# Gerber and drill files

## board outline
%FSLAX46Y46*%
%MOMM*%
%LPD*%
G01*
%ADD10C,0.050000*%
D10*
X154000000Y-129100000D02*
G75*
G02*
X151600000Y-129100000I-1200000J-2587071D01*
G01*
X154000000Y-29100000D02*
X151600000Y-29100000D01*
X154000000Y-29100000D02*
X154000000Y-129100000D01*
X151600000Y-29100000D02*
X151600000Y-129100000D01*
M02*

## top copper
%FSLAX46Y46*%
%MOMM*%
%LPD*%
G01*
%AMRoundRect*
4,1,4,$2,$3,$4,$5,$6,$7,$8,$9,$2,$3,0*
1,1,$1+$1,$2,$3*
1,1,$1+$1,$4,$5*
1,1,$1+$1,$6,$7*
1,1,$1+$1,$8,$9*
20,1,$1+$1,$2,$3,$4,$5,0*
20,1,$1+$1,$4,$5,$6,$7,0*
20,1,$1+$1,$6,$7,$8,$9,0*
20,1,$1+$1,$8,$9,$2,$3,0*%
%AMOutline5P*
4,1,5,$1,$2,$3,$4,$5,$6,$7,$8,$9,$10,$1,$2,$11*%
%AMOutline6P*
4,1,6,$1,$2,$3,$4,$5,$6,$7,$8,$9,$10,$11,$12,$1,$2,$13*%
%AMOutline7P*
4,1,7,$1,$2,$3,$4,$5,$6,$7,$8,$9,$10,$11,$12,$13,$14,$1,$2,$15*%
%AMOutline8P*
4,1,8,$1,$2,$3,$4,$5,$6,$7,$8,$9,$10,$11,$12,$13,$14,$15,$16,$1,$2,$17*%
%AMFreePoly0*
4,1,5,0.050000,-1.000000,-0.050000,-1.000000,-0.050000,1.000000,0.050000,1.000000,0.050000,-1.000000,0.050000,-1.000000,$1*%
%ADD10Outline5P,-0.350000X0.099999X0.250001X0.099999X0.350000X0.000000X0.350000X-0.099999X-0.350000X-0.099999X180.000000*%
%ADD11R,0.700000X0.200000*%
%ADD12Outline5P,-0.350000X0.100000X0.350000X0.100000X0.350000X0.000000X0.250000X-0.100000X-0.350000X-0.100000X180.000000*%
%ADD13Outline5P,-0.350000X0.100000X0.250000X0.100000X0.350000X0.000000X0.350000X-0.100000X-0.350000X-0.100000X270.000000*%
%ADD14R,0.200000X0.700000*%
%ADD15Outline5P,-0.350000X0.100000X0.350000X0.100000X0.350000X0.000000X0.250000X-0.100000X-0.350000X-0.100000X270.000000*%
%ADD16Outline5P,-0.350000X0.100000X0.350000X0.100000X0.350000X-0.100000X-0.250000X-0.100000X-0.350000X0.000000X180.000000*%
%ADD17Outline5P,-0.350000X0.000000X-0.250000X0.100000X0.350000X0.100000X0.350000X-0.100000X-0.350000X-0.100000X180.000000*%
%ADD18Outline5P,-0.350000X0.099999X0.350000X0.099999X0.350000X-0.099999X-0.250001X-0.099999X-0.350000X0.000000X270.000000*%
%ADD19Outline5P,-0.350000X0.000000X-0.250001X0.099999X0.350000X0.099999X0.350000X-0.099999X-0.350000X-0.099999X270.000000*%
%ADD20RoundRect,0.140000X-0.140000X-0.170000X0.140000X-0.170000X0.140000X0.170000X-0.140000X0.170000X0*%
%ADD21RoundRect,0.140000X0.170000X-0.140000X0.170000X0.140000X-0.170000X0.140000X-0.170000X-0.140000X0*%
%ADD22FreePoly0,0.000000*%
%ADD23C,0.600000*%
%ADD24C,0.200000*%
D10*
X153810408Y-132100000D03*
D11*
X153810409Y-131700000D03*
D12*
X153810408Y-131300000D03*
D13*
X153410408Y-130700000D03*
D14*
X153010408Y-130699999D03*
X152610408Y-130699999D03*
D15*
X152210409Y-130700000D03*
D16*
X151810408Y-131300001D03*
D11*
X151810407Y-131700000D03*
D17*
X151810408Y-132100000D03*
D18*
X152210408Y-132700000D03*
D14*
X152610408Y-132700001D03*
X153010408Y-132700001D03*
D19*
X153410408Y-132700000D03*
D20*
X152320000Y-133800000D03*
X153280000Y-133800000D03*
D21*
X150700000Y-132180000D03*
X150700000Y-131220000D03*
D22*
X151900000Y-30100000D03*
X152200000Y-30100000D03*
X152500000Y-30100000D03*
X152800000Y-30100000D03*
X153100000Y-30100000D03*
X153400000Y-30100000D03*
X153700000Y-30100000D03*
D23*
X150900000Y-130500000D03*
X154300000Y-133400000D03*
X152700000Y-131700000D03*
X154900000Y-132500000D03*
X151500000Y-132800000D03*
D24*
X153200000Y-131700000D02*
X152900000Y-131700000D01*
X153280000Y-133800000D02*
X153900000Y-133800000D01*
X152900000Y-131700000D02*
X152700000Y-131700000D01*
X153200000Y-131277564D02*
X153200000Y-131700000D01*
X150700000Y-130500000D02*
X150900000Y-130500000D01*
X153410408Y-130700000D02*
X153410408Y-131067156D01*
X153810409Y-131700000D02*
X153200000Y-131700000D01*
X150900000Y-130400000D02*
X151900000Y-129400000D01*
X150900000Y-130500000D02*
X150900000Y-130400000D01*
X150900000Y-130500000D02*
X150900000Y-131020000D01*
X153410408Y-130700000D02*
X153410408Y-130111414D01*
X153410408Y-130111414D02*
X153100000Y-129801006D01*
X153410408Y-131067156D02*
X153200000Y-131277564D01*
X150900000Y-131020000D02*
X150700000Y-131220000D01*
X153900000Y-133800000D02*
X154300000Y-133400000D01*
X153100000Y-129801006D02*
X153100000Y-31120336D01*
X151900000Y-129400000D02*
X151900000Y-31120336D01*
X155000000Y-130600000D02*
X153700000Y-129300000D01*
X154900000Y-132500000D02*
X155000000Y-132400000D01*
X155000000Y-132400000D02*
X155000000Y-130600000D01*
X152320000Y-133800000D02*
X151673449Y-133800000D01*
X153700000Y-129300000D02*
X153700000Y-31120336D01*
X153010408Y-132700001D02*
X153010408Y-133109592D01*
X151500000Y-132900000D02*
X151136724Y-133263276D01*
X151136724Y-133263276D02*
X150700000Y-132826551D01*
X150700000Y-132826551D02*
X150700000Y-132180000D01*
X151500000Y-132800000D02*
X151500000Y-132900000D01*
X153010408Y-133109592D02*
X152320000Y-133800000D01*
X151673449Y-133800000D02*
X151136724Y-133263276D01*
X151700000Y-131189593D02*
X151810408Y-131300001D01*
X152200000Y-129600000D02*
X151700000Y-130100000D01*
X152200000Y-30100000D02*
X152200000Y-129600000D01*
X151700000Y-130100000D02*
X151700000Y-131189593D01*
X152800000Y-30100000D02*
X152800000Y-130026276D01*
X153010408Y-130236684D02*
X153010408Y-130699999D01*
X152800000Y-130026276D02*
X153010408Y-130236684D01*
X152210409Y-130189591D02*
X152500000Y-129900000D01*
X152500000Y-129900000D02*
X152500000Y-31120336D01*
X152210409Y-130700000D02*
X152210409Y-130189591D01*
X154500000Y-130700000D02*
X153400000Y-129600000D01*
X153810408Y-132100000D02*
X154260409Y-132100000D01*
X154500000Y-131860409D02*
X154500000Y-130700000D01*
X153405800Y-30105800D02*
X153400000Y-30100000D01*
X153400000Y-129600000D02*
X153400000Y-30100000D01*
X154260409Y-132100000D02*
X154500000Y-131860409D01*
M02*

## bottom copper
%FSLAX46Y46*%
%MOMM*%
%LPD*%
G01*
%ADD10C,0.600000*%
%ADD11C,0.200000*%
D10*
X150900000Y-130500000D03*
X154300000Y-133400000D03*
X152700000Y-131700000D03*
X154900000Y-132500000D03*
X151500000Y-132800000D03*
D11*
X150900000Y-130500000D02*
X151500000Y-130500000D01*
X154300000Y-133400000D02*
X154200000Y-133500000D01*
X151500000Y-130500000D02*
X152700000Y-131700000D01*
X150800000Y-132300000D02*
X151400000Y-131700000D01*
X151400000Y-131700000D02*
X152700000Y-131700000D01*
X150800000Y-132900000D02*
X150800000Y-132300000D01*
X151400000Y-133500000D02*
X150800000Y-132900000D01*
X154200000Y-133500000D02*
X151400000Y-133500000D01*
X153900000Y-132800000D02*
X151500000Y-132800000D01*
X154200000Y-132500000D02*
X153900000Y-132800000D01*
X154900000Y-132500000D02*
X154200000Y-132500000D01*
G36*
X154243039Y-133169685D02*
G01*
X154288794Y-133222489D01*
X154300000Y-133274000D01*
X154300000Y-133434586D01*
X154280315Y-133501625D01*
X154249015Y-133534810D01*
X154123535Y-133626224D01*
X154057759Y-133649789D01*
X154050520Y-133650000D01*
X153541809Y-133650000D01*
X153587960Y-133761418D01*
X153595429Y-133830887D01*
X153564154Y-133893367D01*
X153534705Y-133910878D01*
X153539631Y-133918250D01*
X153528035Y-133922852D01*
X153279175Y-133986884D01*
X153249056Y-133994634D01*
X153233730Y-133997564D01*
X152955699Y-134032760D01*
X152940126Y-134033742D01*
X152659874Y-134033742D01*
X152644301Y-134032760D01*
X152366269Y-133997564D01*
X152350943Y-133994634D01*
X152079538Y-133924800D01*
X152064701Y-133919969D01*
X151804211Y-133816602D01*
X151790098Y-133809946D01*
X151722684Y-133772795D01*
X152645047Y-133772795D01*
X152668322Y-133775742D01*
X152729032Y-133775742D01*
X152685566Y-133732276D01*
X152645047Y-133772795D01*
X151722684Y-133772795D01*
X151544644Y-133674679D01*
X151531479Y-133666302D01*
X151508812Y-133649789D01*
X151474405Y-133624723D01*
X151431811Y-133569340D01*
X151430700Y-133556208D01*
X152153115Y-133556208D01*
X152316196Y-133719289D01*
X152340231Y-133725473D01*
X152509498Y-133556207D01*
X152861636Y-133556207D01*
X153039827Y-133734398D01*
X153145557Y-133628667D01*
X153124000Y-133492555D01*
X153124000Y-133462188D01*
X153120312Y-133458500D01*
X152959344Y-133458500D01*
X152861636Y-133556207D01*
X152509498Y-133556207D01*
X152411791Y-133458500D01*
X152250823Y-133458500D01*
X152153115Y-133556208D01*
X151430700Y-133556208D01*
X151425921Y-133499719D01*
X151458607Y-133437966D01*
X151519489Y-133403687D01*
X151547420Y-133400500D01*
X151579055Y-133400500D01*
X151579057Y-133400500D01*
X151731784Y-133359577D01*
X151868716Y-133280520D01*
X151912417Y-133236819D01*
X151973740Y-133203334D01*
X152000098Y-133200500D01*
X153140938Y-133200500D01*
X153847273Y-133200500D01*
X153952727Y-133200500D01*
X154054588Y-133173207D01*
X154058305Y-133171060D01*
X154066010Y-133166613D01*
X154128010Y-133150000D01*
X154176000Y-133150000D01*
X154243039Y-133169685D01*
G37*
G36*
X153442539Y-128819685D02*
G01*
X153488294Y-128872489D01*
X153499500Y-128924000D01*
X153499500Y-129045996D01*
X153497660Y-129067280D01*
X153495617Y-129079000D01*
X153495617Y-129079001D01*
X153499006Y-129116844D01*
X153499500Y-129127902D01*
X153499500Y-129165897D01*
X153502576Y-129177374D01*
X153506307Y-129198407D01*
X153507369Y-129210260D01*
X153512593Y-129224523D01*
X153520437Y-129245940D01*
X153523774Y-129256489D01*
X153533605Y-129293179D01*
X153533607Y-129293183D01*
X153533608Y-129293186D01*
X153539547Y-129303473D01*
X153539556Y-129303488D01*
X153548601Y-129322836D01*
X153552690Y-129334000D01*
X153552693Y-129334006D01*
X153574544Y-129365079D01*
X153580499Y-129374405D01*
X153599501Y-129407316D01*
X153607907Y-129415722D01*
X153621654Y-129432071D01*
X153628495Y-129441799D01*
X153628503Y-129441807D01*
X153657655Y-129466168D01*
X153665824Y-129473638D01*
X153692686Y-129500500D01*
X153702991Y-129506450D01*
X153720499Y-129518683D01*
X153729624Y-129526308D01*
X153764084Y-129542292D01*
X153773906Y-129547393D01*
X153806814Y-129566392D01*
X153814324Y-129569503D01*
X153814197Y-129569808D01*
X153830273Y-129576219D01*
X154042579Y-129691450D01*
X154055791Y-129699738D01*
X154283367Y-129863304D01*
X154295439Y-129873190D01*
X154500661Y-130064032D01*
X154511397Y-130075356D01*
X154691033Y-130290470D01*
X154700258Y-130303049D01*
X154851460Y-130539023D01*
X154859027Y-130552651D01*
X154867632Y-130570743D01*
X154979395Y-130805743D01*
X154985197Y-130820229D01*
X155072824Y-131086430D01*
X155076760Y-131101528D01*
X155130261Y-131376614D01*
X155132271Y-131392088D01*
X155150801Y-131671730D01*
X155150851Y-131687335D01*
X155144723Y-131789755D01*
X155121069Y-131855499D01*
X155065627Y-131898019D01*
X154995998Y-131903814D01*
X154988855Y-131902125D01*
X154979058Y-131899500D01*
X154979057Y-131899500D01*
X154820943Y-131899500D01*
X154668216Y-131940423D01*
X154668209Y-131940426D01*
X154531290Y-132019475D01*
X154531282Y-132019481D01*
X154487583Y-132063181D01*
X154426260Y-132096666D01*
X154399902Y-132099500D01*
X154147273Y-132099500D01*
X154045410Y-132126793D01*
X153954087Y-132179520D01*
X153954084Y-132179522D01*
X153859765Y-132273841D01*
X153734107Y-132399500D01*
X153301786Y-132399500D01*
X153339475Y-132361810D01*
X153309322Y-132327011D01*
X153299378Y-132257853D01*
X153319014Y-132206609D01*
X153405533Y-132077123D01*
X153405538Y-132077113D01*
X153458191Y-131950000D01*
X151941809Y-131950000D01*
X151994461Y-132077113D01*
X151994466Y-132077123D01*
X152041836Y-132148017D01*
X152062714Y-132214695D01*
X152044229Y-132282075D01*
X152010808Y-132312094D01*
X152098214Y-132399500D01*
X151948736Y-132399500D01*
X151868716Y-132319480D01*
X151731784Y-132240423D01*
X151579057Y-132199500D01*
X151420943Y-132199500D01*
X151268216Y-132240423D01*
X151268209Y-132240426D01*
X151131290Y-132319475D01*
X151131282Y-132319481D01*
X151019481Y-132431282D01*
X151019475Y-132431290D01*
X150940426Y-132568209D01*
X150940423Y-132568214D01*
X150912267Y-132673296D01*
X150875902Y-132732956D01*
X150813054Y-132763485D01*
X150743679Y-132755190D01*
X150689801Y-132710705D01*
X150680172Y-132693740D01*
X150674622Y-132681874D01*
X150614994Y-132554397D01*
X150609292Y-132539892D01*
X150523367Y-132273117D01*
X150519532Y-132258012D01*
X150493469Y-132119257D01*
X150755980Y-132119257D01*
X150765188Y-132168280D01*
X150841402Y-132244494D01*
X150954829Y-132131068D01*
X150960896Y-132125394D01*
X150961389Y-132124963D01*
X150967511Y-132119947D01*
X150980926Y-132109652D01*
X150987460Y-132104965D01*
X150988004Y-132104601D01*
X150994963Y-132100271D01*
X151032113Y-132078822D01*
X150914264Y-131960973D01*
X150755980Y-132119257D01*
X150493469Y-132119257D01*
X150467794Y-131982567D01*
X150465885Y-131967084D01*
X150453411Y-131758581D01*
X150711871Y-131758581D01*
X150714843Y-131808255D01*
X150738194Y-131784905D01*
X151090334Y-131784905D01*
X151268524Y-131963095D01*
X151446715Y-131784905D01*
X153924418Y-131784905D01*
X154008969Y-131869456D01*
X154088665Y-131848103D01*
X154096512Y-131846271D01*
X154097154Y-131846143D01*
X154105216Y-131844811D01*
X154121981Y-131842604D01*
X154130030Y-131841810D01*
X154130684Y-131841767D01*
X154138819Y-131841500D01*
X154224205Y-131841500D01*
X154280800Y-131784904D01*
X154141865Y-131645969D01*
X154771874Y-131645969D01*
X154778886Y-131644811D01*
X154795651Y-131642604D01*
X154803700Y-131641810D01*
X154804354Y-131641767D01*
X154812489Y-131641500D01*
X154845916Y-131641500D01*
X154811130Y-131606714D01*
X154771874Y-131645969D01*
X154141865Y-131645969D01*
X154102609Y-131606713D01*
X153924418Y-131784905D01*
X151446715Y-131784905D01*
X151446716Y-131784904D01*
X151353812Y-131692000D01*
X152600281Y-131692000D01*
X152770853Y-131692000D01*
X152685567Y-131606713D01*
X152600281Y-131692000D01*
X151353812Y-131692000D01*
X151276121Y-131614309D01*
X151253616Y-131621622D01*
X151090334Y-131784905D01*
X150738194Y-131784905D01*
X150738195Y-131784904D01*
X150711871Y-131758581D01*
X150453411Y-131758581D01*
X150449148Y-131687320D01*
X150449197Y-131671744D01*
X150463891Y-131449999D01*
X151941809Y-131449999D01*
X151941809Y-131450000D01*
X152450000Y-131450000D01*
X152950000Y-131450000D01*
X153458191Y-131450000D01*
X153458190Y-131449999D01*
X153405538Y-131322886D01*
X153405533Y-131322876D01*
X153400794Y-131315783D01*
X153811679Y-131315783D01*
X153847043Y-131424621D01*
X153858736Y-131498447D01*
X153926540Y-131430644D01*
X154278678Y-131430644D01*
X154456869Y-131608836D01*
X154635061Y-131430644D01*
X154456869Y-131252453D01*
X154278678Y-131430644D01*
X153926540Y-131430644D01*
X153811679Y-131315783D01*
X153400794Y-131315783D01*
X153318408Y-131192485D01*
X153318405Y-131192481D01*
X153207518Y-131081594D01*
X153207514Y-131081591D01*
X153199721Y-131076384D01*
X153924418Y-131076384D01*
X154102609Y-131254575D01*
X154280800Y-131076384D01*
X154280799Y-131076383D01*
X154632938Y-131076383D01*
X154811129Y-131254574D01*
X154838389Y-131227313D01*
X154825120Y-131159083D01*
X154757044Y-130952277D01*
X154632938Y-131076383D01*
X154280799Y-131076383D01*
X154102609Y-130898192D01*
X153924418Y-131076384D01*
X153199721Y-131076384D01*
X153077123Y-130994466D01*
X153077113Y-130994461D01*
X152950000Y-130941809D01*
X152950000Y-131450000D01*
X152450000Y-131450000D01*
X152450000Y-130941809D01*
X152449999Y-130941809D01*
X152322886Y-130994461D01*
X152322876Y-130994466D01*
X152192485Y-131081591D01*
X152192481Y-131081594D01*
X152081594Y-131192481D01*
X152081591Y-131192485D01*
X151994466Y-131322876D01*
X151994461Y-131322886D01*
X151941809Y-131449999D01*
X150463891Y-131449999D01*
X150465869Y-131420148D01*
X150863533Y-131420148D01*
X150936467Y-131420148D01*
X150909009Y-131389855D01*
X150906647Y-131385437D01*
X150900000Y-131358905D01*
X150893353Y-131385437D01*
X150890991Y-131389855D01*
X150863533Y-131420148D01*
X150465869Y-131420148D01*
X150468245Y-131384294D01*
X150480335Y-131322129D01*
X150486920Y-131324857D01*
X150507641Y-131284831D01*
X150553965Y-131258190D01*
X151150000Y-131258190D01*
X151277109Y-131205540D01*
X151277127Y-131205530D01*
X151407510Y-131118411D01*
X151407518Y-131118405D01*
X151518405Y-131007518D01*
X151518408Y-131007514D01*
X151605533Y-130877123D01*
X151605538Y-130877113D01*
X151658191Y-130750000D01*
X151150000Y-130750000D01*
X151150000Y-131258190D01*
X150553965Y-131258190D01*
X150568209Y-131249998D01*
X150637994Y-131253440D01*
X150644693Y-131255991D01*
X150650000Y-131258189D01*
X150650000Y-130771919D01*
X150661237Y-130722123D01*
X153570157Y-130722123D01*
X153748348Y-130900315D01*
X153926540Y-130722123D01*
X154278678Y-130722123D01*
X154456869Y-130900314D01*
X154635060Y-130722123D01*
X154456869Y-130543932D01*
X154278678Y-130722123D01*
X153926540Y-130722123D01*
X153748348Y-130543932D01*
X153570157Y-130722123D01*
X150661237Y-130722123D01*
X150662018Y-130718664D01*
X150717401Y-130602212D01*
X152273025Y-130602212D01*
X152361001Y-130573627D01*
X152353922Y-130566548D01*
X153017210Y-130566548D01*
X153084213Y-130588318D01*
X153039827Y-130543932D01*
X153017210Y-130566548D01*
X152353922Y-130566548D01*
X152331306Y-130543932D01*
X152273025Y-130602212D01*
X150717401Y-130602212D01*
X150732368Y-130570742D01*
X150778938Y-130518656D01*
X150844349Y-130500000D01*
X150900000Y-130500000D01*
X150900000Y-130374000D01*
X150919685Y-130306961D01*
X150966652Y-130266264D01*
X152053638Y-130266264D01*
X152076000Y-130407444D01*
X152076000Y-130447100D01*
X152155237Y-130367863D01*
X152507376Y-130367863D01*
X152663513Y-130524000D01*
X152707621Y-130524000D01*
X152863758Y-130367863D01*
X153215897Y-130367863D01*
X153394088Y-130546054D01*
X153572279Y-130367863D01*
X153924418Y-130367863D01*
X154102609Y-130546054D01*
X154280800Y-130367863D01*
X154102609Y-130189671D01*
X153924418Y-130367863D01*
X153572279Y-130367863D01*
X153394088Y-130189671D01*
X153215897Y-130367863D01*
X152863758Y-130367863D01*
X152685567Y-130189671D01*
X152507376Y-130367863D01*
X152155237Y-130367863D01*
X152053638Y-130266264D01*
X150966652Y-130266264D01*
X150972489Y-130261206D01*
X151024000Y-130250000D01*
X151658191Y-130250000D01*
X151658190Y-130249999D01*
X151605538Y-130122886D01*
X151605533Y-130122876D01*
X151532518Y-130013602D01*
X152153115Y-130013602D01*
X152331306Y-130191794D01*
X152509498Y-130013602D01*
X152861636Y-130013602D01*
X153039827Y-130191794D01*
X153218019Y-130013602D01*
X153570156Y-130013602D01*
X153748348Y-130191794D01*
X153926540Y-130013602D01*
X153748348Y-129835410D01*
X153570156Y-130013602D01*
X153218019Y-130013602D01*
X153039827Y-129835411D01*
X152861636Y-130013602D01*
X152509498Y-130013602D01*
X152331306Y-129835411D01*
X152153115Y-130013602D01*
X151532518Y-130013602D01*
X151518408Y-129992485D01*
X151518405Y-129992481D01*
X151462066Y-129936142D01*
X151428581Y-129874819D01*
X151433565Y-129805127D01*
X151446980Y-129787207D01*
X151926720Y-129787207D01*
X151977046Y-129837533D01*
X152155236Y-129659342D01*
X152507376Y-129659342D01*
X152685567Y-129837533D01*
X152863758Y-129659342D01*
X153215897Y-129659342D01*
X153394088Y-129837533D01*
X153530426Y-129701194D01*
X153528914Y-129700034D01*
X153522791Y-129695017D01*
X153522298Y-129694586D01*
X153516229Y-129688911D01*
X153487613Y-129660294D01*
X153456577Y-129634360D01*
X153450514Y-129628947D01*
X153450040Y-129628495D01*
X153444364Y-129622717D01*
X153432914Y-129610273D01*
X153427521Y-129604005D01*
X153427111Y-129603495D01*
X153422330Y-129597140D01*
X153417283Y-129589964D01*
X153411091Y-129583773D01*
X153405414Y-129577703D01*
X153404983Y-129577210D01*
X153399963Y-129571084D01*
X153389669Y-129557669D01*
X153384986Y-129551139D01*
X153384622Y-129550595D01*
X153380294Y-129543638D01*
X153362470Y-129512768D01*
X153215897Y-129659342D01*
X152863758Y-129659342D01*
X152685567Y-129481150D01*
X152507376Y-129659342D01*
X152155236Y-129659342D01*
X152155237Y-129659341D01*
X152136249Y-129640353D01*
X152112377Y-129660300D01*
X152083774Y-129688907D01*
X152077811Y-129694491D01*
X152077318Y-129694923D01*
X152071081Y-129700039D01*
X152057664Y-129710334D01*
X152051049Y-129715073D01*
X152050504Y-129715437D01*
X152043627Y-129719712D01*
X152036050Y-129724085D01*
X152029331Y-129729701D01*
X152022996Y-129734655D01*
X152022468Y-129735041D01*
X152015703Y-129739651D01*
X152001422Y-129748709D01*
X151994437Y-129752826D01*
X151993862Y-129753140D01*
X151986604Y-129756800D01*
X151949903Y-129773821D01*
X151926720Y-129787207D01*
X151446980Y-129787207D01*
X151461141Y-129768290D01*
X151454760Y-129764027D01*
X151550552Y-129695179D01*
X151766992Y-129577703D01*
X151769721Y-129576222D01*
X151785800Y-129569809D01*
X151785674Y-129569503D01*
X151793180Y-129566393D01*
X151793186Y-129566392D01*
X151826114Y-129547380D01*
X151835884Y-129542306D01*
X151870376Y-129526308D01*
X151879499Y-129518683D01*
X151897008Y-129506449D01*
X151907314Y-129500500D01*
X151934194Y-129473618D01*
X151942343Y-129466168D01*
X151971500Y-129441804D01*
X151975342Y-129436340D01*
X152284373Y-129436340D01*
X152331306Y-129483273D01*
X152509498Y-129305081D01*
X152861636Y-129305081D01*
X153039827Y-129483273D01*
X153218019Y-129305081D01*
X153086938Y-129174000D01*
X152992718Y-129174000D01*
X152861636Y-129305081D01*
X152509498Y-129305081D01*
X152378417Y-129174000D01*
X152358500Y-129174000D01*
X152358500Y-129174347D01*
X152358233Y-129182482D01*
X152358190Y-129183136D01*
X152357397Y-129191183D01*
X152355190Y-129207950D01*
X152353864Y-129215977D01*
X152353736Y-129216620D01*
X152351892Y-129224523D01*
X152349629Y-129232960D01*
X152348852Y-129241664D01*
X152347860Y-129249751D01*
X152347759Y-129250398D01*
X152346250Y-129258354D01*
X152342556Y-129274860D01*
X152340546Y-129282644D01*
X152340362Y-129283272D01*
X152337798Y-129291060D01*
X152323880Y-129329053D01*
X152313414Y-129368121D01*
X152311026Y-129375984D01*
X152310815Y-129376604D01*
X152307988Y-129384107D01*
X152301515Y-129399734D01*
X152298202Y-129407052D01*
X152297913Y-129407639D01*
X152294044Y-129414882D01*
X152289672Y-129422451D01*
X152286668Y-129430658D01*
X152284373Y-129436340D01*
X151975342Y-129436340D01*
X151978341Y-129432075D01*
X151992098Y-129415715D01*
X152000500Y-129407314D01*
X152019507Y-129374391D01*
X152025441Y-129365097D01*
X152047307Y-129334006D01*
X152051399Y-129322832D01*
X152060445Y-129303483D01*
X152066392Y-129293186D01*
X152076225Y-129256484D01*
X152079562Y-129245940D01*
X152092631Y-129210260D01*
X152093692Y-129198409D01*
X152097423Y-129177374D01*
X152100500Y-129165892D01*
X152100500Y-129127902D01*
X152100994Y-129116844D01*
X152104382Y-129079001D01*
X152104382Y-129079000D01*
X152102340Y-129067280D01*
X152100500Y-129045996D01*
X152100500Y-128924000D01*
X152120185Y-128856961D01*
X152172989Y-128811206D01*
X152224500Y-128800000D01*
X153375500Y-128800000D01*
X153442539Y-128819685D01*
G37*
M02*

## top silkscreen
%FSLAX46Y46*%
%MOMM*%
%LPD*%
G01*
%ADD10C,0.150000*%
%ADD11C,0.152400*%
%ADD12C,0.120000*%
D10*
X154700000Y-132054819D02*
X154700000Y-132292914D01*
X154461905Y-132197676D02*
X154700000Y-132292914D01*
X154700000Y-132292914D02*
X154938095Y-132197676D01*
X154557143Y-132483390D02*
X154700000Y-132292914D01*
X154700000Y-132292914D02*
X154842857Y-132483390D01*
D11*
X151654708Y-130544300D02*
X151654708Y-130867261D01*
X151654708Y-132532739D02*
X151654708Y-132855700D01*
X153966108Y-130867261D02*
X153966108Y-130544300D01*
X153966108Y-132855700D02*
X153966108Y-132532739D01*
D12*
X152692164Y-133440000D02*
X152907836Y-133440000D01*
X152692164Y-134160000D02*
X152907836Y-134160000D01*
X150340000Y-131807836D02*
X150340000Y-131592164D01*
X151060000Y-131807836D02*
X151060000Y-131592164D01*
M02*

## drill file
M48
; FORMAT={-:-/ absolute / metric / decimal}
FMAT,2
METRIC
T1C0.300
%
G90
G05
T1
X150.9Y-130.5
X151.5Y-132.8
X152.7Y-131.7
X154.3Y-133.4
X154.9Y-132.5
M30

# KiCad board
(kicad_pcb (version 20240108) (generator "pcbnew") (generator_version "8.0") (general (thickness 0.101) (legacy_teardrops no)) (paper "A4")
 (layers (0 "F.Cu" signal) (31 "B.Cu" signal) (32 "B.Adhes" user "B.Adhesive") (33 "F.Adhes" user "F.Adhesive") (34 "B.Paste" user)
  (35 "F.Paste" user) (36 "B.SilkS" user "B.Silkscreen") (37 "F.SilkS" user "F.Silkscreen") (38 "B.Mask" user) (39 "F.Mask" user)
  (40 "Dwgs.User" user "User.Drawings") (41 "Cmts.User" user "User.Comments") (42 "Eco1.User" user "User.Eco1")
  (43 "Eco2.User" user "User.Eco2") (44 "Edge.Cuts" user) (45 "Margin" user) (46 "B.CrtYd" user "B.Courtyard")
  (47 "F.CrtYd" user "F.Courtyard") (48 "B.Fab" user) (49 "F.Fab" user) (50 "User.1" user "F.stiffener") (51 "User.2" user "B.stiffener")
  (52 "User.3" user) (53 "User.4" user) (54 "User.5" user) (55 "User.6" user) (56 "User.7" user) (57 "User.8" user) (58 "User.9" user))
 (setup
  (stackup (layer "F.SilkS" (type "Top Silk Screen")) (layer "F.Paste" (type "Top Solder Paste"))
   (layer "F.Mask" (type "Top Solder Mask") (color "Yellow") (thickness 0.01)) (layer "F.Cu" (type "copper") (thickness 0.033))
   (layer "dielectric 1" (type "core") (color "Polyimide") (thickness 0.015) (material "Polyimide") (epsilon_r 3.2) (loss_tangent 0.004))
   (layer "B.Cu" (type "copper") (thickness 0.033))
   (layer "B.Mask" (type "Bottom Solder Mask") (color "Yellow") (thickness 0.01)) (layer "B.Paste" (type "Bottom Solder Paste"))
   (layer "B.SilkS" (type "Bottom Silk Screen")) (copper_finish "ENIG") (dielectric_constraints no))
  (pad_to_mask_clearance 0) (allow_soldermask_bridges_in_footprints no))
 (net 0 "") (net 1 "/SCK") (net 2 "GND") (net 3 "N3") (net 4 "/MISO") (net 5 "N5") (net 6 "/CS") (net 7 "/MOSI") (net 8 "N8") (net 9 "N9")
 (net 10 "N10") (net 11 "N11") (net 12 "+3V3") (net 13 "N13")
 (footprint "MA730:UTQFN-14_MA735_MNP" (layer "F.Cu") (at 152.810408 131.7 180)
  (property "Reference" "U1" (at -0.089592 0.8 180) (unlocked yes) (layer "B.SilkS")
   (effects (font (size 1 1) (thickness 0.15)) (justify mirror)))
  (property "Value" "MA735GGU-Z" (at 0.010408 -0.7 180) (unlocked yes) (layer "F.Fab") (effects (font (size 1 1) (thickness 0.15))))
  (fp_line (start 1.1557 1.1557) (end 1.1557 0.832739) (stroke (width 0.1524) (type solid)) (layer "F.SilkS"))
  (fp_line (start 1.1557 -0.832739) (end 1.1557 -1.1557) (stroke (width 0.1524) (type solid)) (layer "F.SilkS"))
  (fp_line (start -1.1557 0.832739) (end -1.1557 1.1557) (stroke (width 0.1524) (type solid)) (layer "F.SilkS"))
  (fp_line (start -1.1557 -1.1557) (end -1.1557 -0.832739) (stroke (width 0.1524) (type solid)) (layer "F.SilkS"))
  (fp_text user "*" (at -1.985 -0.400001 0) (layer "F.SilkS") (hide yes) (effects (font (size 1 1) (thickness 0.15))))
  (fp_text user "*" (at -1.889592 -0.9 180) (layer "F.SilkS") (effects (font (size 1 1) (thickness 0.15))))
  (pad "1" smd roundrect (at -1 -0.4 180) (size 0.7 0.199998) (layers "F.Cu" "F.Paste" "F.Mask") (roundrect_rratio 0) (chamfer_ratio 0.5)
   (chamfer top_right) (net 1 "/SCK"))
  (pad "2" smd rect (at -1.000001 0 180) (size 0.7 0.2) (layers "F.Cu" "F.Paste" "F.Mask") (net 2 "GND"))
  (pad "3" smd roundrect (at -1 0.4 180) (size 0.7 0.2) (layers "F.Cu" "F.Paste" "F.Mask") (roundrect_rratio 0) (chamfer_ratio 0.5)
   (chamfer bottom_right) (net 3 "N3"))
  (pad "4" smd roundrect (at -0.6 1 270) (size 0.7 0.2) (layers "F.Cu" "F.Paste" "F.Mask") (roundrect_rratio 0) (chamfer_ratio 0.5)
   (chamfer top_right) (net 2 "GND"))
  (pad "5" smd rect (at -0.2 1.000001 270) (size 0.7 0.2) (layers "F.Cu" "F.Paste" "F.Mask") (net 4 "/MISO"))
  (pad "6" smd rect (at 0.2 1.000001 270) (size 0.7 0.2) (layers "F.Cu" "F.Paste" "F.Mask") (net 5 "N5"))
  (pad "7" smd roundrect (at 0.599999 1 270) (size 0.7 0.199999) (layers "F.Cu" "F.Paste" "F.Mask") (roundrect_rratio 0) (chamfer_ratio 0.5)
   (chamfer bottom_right) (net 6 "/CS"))
  (pad "8" smd roundrect (at 1 0.399999 180) (size 0.7 0.2) (layers "F.Cu" "F.Paste" "F.Mask") (roundrect_rratio 0) (chamfer_ratio 0.5)
   (chamfer bottom_left) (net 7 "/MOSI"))
  (pad "9" smd rect (at 1.000001 0 180) (size 0.7 0.2) (layers "F.Cu" "F.Paste" "F.Mask") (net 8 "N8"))
  (pad "10" smd roundrect (at 1 -0.4 180) (size 0.7 0.2) (layers "F.Cu" "F.Paste" "F.Mask") (roundrect_rratio 0) (chamfer_ratio 0.5)
   (chamfer top_left) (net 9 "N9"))
  (pad "11" smd roundrect (at 0.6 -1 270) (size 0.7 0.199998) (layers "F.Cu" "F.Paste" "F.Mask") (roundrect_rratio 0) (chamfer_ratio 0.5)
   (chamfer bottom_left) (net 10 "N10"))
  (pad "12" smd rect (at 0.2 -1.000001 270) (size 0.7 0.2) (layers "F.Cu" "F.Paste" "F.Mask") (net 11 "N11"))
  (pad "13" smd rect (at -0.2 -1.000001 270) (size 0.7 0.2) (layers "F.Cu" "F.Paste" "F.Mask") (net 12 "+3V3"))
  (pad "14" smd roundrect (at -0.6 -1 270) (size 0.7 0.199998) (layers "F.Cu" "F.Paste" "F.Mask") (roundrect_rratio 0) (chamfer_ratio 0.5)
   (chamfer top_left) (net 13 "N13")))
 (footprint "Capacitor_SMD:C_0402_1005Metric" (layer "F.Cu") (at 152.8 133.8)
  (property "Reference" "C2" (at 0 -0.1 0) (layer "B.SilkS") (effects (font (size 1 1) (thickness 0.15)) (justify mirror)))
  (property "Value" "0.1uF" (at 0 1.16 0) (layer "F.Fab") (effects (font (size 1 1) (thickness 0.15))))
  (fp_line (start -0.107836 -0.36) (end 0.107836 -0.36) (stroke (width 0.12) (type solid)) (layer "F.SilkS"))
  (fp_line (start -0.107836 0.36) (end 0.107836 0.36) (stroke (width 0.12) (type solid)) (layer "F.SilkS"))
  (pad "1" smd roundrect (at -0.48 0) (size 0.56 0.62) (layers "F.Cu" "F.Paste" "F.Mask") (roundrect_rratio 0.25) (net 12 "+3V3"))
  (pad "2" smd roundrect (at 0.48 0) (size 0.56 0.62) (layers "F.Cu" "F.Paste" "F.Mask") (roundrect_rratio 0.25) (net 2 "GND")))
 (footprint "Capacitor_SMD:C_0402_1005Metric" (layer "F.Cu") (at 150.7 131.7 90)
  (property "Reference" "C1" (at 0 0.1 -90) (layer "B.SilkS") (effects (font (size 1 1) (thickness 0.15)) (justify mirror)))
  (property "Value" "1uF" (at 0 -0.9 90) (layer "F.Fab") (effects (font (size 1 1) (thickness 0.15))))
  (fp_line (start -0.107836 -0.36) (end 0.107836 -0.36) (stroke (width 0.12) (type solid)) (layer "F.SilkS"))
  (fp_line (start -0.107836 0.36) (end 0.107836 0.36) (stroke (width 0.12) (type solid)) (layer "F.SilkS"))
  (pad "1" smd roundrect (at -0.48 0 90) (size 0.56 0.62) (layers "F.Cu" "F.Paste" "F.Mask") (roundrect_rratio 0.25) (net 12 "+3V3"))
  (pad "2" smd roundrect (at 0.48 0 90) (size 0.56 0.62) (layers "F.Cu" "F.Paste" "F.Mask") (roundrect_rratio 0.25) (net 2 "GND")))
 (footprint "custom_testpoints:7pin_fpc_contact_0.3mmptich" (layer "F.Cu") (at 152.8 30.2)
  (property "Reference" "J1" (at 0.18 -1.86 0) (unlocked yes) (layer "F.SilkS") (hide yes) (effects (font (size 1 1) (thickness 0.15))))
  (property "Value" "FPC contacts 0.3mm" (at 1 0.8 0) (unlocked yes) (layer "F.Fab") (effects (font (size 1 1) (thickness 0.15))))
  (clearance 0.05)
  (pad "1" connect custom (at -0.9 -0.1) (size 0.1 2) (layers "F.Cu" "F.Mask") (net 2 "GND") (clearance 0.05)
   (options (clearance outline) (anchor rect)) (primitives))
  (pad "2" connect custom (at -0.6 -0.1) (size 0.1 2) (layers "F.Cu" "F.Mask") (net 7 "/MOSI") (clearance 0.05)
   (options (clearance outline) (anchor rect)) (primitives))
  (pad "3" connect custom (at -0.3 -0.1) (size 0.1 2) (layers "F.Cu" "F.Mask") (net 6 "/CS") (clearance 0.05)
   (options (clearance outline) (anchor rect)) (primitives))
  (pad "4" connect custom (at 0 -0.1) (size 0.1 2) (layers "F.Cu" "F.Mask") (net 4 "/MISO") (clearance 0.05)
   (options (clearance outline) (anchor rect)) (primitives))
  (pad "5" connect custom (at 0.3 -0.1) (size 0.1 2) (layers "F.Cu" "F.Mask") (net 2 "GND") (clearance 0.05)
   (options (clearance outline) (anchor rect)) (primitives))
  (pad "6" connect custom (at 0.6 -0.1) (size 0.1 2) (layers "F.Cu" "F.Mask") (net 1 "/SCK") (clearance 0.05)
   (options (clearance outline) (anchor rect)) (primitives))
  (pad "7" connect custom (at 0.9 -0.1) (size 0.1 2) (layers "F.Cu" "F.Mask") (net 12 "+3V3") (clearance 0.05)
   (options (clearance outline) (anchor rect)) (primitives)))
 (gr_arc (start 154 129.1) (mid 152.8 134.538901) (end 151.6 129.1) (stroke (width 0.05) (type default)) (layer "Edge.Cuts"))
 (gr_line (start 154 29.1) (end 151.6 29.1) (stroke (width 0.05) (type default)) (layer "Edge.Cuts"))
 (gr_line (start 154 29.1) (end 154 129.1) (stroke (width 0.05) (type default)) (layer "Edge.Cuts"))
 (gr_line (start 151.6 29.1) (end 151.6 129.1) (stroke (width 0.05) (type default)) (layer "Edge.Cuts"))
 (segment (start 153.2 131.7) (end 152.9 131.7) (width 0.2) (layer "F.Cu") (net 2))
 (segment (start 153.28 133.8) (end 153.9 133.8) (width 0.2) (layer "F.Cu") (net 2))
 (segment (start 152.9 131.7) (end 152.7 131.7) (width 0.2) (layer "F.Cu") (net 2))
 (segment (start 153.2 131.277564) (end 153.2 131.7) (width 0.2) (layer "F.Cu") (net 2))
 (segment (start 150.7 130.5) (end 150.9 130.5) (width 0.2) (layer "F.Cu") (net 2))
 (segment (start 153.410408 130.7) (end 153.410408 131.067156) (width 0.2) (layer "F.Cu") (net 2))
 (segment (start 153.810409 131.7) (end 153.2 131.7) (width 0.2) (layer "F.Cu") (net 2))
 (segment (start 150.9 130.4) (end 151.9 129.4) (width 0.2) (layer "F.Cu") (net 2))
 (segment (start 150.9 130.5) (end 150.9 130.4) (width 0.2) (layer "F.Cu") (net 2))
 (segment (start 150.9 130.5) (end 150.9 131.02) (width 0.2) (layer "F.Cu") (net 2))
 (segment (start 153.410408 130.7) (end 153.410408 130.111414) (width 0.2) (layer "F.Cu") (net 2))
 (segment (start 153.410408 130.111414) (end 153.1 129.801006) (width 0.2) (layer "F.Cu") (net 2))
 (segment (start 153.410408 131.067156) (end 153.2 131.277564) (width 0.2) (layer "F.Cu") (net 2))
 (segment (start 150.9 131.02) (end 150.7 131.22) (width 0.2) (layer "F.Cu") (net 2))
 (segment (start 153.9 133.8) (end 154.3 133.4) (width 0.2) (layer "F.Cu") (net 2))
 (segment (start 153.1 129.801006) (end 153.1 31.120336) (width 0.2) (layer "F.Cu") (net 2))
 (segment (start 151.9 129.4) (end 151.9 31.120336) (width 0.2) (layer "F.Cu") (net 2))
 (via (at 150.9 130.5) (size 0.6) (drill 0.3) (layers "F.Cu" "B.Cu") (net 2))
 (via (at 154.3 133.4) (size 0.6) (drill 0.3) (layers "F.Cu" "B.Cu") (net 2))
 (via (at 152.7 131.7) (size 0.6) (drill 0.3) (layers "F.Cu" "B.Cu") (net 2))
 (segment (start 150.9 130.5) (end 151.5 130.5) (width 0.2) (layer "B.Cu") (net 2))
 (segment (start 154.3 133.4) (end 154.2 133.5) (width 0.2) (layer "B.Cu") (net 2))
 (segment (start 151.5 130.5) (end 152.7 131.7) (width 0.2) (layer "B.Cu") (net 2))
 (segment (start 150.8 132.3) (end 151.4 131.7) (width 0.2) (layer "B.Cu") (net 2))
 (segment (start 151.4 131.7) (end 152.7 131.7) (width 0.2) (layer "B.Cu") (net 2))
 (segment (start 150.8 132.9) (end 150.8 132.3) (width 0.2) (layer "B.Cu") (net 2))
 (segment (start 151.4 133.5) (end 150.8 132.9) (width 0.2) (layer "B.Cu") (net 2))
 (segment (start 154.2 133.5) (end 151.4 133.5) (width 0.2) (layer "B.Cu") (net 2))
 (segment (start 155 130.6) (end 153.7 129.3) (width 0.2) (layer "F.Cu") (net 12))
 (segment (start 154.9 132.5) (end 155 132.4) (width 0.2) (layer "F.Cu") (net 12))
 (segment (start 155 132.4) (end 155 130.6) (width 0.2) (layer "F.Cu") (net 12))
 (segment (start 152.32 133.8) (end 151.673449 133.8) (width 0.2) (layer "F.Cu") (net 12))
 (segment (start 153.7 129.3) (end 153.7 31.120336) (width 0.2) (layer "F.Cu") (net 12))
 (segment (start 153.010408 132.700001) (end 153.010408 133.109592) (width 0.2) (layer "F.Cu") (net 12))
 (segment (start 151.5 132.9) (end 151.136724 133.263276) (width 0.2) (layer "F.Cu") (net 12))
 (segment (start 151.136724 133.263276) (end 150.7 132.826551) (width 0.2) (layer "F.Cu") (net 12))
 (segment (start 150.7 132.826551) (end 150.7 132.18) (width 0.2) (layer "F.Cu") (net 12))
 (segment (start 151.5 132.8) (end 151.5 132.9) (width 0.2) (layer "F.Cu") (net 12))
 (segment (start 153.010408 133.109592) (end 152.32 133.8) (width 0.2) (layer "F.Cu") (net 12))
 (segment (start 151.673449 133.8) (end 151.136724 133.263276) (width 0.2) (layer "F.Cu") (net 12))
 (via (at 154.9 132.5) (size 0.6) (drill 0.3) (layers "F.Cu" "B.Cu") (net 12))
 (via (at 151.5 132.8) (size 0.6) (drill 0.3) (layers "F.Cu" "B.Cu") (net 12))
 (segment (start 153.9 132.8) (end 151.5 132.8) (width 0.2) (layer "B.Cu") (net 12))
 (segment (start 154.2 132.5) (end 153.9 132.8) (width 0.2) (layer "B.Cu") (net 12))
 (segment (start 154.9 132.5) (end 154.2 132.5) (width 0.2) (layer "B.Cu") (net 12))
 (segment (start 151.7 131.189593) (end 151.810408 131.300001) (width 0.2) (layer "F.Cu") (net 7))
 (segment (start 152.2 129.6) (end 151.7 130.1) (width 0.2) (layer "F.Cu") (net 7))
 (segment (start 152.2 30.1) (end 152.2 129.6) (width 0.2) (layer "F.Cu") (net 7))
 (segment (start 151.7 130.1) (end 151.7 131.189593) (width 0.2) (layer "F.Cu") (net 7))
 (segment (start 152.8 30.1) (end 152.8 130.026276) (width 0.2) (layer "F.Cu") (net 4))
 (segment (start 153.010408 130.236684) (end 153.010408 130.699999) (width 0.2) (layer "F.Cu") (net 4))
 (segment (start 152.8 130.026276) (end 153.010408 130.236684) (width 0.2) (layer "F.Cu") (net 4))
 (segment (start 152.210409 130.189591) (end 152.5 129.9) (width 0.2) (layer "F.Cu") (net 6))
 (segment (start 152.5 129.9) (end 152.5 31.120336) (width 0.2) (layer "F.Cu") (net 6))
 (segment (start 152.210409 130.7) (end 152.210409 130.189591) (width 0.2) (layer "F.Cu") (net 6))
 (segment (start 154.5 130.7) (end 153.4 129.6) (width 0.2) (layer "F.Cu") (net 1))
 (segment (start 153.810408 132.1) (end 154.260409 132.1) (width 0.2) (layer "F.Cu") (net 1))
 (segment (start 154.5 131.860409) (end 154.5 130.7) (width 0.2) (layer "F.Cu") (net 1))
 (segment (start 153.4058 30.1058) (end 153.4 30.1) (width 0.2) (layer "F.Cu") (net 1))
 (segment (start 153.4 129.6) (end 153.4 30.1) (width 0.2) (layer "F.Cu") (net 1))
 (segment (start 154.260409 132.1) (end 154.5 131.860409) (width 0.2) (layer "F.Cu") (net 1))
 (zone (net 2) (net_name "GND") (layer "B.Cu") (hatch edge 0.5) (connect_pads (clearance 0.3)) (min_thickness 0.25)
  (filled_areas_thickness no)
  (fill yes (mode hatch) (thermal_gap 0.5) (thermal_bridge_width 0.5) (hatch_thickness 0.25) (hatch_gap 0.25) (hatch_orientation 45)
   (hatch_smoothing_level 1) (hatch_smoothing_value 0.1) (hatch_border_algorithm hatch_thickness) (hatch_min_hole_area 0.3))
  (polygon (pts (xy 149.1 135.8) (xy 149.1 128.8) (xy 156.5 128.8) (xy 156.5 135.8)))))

